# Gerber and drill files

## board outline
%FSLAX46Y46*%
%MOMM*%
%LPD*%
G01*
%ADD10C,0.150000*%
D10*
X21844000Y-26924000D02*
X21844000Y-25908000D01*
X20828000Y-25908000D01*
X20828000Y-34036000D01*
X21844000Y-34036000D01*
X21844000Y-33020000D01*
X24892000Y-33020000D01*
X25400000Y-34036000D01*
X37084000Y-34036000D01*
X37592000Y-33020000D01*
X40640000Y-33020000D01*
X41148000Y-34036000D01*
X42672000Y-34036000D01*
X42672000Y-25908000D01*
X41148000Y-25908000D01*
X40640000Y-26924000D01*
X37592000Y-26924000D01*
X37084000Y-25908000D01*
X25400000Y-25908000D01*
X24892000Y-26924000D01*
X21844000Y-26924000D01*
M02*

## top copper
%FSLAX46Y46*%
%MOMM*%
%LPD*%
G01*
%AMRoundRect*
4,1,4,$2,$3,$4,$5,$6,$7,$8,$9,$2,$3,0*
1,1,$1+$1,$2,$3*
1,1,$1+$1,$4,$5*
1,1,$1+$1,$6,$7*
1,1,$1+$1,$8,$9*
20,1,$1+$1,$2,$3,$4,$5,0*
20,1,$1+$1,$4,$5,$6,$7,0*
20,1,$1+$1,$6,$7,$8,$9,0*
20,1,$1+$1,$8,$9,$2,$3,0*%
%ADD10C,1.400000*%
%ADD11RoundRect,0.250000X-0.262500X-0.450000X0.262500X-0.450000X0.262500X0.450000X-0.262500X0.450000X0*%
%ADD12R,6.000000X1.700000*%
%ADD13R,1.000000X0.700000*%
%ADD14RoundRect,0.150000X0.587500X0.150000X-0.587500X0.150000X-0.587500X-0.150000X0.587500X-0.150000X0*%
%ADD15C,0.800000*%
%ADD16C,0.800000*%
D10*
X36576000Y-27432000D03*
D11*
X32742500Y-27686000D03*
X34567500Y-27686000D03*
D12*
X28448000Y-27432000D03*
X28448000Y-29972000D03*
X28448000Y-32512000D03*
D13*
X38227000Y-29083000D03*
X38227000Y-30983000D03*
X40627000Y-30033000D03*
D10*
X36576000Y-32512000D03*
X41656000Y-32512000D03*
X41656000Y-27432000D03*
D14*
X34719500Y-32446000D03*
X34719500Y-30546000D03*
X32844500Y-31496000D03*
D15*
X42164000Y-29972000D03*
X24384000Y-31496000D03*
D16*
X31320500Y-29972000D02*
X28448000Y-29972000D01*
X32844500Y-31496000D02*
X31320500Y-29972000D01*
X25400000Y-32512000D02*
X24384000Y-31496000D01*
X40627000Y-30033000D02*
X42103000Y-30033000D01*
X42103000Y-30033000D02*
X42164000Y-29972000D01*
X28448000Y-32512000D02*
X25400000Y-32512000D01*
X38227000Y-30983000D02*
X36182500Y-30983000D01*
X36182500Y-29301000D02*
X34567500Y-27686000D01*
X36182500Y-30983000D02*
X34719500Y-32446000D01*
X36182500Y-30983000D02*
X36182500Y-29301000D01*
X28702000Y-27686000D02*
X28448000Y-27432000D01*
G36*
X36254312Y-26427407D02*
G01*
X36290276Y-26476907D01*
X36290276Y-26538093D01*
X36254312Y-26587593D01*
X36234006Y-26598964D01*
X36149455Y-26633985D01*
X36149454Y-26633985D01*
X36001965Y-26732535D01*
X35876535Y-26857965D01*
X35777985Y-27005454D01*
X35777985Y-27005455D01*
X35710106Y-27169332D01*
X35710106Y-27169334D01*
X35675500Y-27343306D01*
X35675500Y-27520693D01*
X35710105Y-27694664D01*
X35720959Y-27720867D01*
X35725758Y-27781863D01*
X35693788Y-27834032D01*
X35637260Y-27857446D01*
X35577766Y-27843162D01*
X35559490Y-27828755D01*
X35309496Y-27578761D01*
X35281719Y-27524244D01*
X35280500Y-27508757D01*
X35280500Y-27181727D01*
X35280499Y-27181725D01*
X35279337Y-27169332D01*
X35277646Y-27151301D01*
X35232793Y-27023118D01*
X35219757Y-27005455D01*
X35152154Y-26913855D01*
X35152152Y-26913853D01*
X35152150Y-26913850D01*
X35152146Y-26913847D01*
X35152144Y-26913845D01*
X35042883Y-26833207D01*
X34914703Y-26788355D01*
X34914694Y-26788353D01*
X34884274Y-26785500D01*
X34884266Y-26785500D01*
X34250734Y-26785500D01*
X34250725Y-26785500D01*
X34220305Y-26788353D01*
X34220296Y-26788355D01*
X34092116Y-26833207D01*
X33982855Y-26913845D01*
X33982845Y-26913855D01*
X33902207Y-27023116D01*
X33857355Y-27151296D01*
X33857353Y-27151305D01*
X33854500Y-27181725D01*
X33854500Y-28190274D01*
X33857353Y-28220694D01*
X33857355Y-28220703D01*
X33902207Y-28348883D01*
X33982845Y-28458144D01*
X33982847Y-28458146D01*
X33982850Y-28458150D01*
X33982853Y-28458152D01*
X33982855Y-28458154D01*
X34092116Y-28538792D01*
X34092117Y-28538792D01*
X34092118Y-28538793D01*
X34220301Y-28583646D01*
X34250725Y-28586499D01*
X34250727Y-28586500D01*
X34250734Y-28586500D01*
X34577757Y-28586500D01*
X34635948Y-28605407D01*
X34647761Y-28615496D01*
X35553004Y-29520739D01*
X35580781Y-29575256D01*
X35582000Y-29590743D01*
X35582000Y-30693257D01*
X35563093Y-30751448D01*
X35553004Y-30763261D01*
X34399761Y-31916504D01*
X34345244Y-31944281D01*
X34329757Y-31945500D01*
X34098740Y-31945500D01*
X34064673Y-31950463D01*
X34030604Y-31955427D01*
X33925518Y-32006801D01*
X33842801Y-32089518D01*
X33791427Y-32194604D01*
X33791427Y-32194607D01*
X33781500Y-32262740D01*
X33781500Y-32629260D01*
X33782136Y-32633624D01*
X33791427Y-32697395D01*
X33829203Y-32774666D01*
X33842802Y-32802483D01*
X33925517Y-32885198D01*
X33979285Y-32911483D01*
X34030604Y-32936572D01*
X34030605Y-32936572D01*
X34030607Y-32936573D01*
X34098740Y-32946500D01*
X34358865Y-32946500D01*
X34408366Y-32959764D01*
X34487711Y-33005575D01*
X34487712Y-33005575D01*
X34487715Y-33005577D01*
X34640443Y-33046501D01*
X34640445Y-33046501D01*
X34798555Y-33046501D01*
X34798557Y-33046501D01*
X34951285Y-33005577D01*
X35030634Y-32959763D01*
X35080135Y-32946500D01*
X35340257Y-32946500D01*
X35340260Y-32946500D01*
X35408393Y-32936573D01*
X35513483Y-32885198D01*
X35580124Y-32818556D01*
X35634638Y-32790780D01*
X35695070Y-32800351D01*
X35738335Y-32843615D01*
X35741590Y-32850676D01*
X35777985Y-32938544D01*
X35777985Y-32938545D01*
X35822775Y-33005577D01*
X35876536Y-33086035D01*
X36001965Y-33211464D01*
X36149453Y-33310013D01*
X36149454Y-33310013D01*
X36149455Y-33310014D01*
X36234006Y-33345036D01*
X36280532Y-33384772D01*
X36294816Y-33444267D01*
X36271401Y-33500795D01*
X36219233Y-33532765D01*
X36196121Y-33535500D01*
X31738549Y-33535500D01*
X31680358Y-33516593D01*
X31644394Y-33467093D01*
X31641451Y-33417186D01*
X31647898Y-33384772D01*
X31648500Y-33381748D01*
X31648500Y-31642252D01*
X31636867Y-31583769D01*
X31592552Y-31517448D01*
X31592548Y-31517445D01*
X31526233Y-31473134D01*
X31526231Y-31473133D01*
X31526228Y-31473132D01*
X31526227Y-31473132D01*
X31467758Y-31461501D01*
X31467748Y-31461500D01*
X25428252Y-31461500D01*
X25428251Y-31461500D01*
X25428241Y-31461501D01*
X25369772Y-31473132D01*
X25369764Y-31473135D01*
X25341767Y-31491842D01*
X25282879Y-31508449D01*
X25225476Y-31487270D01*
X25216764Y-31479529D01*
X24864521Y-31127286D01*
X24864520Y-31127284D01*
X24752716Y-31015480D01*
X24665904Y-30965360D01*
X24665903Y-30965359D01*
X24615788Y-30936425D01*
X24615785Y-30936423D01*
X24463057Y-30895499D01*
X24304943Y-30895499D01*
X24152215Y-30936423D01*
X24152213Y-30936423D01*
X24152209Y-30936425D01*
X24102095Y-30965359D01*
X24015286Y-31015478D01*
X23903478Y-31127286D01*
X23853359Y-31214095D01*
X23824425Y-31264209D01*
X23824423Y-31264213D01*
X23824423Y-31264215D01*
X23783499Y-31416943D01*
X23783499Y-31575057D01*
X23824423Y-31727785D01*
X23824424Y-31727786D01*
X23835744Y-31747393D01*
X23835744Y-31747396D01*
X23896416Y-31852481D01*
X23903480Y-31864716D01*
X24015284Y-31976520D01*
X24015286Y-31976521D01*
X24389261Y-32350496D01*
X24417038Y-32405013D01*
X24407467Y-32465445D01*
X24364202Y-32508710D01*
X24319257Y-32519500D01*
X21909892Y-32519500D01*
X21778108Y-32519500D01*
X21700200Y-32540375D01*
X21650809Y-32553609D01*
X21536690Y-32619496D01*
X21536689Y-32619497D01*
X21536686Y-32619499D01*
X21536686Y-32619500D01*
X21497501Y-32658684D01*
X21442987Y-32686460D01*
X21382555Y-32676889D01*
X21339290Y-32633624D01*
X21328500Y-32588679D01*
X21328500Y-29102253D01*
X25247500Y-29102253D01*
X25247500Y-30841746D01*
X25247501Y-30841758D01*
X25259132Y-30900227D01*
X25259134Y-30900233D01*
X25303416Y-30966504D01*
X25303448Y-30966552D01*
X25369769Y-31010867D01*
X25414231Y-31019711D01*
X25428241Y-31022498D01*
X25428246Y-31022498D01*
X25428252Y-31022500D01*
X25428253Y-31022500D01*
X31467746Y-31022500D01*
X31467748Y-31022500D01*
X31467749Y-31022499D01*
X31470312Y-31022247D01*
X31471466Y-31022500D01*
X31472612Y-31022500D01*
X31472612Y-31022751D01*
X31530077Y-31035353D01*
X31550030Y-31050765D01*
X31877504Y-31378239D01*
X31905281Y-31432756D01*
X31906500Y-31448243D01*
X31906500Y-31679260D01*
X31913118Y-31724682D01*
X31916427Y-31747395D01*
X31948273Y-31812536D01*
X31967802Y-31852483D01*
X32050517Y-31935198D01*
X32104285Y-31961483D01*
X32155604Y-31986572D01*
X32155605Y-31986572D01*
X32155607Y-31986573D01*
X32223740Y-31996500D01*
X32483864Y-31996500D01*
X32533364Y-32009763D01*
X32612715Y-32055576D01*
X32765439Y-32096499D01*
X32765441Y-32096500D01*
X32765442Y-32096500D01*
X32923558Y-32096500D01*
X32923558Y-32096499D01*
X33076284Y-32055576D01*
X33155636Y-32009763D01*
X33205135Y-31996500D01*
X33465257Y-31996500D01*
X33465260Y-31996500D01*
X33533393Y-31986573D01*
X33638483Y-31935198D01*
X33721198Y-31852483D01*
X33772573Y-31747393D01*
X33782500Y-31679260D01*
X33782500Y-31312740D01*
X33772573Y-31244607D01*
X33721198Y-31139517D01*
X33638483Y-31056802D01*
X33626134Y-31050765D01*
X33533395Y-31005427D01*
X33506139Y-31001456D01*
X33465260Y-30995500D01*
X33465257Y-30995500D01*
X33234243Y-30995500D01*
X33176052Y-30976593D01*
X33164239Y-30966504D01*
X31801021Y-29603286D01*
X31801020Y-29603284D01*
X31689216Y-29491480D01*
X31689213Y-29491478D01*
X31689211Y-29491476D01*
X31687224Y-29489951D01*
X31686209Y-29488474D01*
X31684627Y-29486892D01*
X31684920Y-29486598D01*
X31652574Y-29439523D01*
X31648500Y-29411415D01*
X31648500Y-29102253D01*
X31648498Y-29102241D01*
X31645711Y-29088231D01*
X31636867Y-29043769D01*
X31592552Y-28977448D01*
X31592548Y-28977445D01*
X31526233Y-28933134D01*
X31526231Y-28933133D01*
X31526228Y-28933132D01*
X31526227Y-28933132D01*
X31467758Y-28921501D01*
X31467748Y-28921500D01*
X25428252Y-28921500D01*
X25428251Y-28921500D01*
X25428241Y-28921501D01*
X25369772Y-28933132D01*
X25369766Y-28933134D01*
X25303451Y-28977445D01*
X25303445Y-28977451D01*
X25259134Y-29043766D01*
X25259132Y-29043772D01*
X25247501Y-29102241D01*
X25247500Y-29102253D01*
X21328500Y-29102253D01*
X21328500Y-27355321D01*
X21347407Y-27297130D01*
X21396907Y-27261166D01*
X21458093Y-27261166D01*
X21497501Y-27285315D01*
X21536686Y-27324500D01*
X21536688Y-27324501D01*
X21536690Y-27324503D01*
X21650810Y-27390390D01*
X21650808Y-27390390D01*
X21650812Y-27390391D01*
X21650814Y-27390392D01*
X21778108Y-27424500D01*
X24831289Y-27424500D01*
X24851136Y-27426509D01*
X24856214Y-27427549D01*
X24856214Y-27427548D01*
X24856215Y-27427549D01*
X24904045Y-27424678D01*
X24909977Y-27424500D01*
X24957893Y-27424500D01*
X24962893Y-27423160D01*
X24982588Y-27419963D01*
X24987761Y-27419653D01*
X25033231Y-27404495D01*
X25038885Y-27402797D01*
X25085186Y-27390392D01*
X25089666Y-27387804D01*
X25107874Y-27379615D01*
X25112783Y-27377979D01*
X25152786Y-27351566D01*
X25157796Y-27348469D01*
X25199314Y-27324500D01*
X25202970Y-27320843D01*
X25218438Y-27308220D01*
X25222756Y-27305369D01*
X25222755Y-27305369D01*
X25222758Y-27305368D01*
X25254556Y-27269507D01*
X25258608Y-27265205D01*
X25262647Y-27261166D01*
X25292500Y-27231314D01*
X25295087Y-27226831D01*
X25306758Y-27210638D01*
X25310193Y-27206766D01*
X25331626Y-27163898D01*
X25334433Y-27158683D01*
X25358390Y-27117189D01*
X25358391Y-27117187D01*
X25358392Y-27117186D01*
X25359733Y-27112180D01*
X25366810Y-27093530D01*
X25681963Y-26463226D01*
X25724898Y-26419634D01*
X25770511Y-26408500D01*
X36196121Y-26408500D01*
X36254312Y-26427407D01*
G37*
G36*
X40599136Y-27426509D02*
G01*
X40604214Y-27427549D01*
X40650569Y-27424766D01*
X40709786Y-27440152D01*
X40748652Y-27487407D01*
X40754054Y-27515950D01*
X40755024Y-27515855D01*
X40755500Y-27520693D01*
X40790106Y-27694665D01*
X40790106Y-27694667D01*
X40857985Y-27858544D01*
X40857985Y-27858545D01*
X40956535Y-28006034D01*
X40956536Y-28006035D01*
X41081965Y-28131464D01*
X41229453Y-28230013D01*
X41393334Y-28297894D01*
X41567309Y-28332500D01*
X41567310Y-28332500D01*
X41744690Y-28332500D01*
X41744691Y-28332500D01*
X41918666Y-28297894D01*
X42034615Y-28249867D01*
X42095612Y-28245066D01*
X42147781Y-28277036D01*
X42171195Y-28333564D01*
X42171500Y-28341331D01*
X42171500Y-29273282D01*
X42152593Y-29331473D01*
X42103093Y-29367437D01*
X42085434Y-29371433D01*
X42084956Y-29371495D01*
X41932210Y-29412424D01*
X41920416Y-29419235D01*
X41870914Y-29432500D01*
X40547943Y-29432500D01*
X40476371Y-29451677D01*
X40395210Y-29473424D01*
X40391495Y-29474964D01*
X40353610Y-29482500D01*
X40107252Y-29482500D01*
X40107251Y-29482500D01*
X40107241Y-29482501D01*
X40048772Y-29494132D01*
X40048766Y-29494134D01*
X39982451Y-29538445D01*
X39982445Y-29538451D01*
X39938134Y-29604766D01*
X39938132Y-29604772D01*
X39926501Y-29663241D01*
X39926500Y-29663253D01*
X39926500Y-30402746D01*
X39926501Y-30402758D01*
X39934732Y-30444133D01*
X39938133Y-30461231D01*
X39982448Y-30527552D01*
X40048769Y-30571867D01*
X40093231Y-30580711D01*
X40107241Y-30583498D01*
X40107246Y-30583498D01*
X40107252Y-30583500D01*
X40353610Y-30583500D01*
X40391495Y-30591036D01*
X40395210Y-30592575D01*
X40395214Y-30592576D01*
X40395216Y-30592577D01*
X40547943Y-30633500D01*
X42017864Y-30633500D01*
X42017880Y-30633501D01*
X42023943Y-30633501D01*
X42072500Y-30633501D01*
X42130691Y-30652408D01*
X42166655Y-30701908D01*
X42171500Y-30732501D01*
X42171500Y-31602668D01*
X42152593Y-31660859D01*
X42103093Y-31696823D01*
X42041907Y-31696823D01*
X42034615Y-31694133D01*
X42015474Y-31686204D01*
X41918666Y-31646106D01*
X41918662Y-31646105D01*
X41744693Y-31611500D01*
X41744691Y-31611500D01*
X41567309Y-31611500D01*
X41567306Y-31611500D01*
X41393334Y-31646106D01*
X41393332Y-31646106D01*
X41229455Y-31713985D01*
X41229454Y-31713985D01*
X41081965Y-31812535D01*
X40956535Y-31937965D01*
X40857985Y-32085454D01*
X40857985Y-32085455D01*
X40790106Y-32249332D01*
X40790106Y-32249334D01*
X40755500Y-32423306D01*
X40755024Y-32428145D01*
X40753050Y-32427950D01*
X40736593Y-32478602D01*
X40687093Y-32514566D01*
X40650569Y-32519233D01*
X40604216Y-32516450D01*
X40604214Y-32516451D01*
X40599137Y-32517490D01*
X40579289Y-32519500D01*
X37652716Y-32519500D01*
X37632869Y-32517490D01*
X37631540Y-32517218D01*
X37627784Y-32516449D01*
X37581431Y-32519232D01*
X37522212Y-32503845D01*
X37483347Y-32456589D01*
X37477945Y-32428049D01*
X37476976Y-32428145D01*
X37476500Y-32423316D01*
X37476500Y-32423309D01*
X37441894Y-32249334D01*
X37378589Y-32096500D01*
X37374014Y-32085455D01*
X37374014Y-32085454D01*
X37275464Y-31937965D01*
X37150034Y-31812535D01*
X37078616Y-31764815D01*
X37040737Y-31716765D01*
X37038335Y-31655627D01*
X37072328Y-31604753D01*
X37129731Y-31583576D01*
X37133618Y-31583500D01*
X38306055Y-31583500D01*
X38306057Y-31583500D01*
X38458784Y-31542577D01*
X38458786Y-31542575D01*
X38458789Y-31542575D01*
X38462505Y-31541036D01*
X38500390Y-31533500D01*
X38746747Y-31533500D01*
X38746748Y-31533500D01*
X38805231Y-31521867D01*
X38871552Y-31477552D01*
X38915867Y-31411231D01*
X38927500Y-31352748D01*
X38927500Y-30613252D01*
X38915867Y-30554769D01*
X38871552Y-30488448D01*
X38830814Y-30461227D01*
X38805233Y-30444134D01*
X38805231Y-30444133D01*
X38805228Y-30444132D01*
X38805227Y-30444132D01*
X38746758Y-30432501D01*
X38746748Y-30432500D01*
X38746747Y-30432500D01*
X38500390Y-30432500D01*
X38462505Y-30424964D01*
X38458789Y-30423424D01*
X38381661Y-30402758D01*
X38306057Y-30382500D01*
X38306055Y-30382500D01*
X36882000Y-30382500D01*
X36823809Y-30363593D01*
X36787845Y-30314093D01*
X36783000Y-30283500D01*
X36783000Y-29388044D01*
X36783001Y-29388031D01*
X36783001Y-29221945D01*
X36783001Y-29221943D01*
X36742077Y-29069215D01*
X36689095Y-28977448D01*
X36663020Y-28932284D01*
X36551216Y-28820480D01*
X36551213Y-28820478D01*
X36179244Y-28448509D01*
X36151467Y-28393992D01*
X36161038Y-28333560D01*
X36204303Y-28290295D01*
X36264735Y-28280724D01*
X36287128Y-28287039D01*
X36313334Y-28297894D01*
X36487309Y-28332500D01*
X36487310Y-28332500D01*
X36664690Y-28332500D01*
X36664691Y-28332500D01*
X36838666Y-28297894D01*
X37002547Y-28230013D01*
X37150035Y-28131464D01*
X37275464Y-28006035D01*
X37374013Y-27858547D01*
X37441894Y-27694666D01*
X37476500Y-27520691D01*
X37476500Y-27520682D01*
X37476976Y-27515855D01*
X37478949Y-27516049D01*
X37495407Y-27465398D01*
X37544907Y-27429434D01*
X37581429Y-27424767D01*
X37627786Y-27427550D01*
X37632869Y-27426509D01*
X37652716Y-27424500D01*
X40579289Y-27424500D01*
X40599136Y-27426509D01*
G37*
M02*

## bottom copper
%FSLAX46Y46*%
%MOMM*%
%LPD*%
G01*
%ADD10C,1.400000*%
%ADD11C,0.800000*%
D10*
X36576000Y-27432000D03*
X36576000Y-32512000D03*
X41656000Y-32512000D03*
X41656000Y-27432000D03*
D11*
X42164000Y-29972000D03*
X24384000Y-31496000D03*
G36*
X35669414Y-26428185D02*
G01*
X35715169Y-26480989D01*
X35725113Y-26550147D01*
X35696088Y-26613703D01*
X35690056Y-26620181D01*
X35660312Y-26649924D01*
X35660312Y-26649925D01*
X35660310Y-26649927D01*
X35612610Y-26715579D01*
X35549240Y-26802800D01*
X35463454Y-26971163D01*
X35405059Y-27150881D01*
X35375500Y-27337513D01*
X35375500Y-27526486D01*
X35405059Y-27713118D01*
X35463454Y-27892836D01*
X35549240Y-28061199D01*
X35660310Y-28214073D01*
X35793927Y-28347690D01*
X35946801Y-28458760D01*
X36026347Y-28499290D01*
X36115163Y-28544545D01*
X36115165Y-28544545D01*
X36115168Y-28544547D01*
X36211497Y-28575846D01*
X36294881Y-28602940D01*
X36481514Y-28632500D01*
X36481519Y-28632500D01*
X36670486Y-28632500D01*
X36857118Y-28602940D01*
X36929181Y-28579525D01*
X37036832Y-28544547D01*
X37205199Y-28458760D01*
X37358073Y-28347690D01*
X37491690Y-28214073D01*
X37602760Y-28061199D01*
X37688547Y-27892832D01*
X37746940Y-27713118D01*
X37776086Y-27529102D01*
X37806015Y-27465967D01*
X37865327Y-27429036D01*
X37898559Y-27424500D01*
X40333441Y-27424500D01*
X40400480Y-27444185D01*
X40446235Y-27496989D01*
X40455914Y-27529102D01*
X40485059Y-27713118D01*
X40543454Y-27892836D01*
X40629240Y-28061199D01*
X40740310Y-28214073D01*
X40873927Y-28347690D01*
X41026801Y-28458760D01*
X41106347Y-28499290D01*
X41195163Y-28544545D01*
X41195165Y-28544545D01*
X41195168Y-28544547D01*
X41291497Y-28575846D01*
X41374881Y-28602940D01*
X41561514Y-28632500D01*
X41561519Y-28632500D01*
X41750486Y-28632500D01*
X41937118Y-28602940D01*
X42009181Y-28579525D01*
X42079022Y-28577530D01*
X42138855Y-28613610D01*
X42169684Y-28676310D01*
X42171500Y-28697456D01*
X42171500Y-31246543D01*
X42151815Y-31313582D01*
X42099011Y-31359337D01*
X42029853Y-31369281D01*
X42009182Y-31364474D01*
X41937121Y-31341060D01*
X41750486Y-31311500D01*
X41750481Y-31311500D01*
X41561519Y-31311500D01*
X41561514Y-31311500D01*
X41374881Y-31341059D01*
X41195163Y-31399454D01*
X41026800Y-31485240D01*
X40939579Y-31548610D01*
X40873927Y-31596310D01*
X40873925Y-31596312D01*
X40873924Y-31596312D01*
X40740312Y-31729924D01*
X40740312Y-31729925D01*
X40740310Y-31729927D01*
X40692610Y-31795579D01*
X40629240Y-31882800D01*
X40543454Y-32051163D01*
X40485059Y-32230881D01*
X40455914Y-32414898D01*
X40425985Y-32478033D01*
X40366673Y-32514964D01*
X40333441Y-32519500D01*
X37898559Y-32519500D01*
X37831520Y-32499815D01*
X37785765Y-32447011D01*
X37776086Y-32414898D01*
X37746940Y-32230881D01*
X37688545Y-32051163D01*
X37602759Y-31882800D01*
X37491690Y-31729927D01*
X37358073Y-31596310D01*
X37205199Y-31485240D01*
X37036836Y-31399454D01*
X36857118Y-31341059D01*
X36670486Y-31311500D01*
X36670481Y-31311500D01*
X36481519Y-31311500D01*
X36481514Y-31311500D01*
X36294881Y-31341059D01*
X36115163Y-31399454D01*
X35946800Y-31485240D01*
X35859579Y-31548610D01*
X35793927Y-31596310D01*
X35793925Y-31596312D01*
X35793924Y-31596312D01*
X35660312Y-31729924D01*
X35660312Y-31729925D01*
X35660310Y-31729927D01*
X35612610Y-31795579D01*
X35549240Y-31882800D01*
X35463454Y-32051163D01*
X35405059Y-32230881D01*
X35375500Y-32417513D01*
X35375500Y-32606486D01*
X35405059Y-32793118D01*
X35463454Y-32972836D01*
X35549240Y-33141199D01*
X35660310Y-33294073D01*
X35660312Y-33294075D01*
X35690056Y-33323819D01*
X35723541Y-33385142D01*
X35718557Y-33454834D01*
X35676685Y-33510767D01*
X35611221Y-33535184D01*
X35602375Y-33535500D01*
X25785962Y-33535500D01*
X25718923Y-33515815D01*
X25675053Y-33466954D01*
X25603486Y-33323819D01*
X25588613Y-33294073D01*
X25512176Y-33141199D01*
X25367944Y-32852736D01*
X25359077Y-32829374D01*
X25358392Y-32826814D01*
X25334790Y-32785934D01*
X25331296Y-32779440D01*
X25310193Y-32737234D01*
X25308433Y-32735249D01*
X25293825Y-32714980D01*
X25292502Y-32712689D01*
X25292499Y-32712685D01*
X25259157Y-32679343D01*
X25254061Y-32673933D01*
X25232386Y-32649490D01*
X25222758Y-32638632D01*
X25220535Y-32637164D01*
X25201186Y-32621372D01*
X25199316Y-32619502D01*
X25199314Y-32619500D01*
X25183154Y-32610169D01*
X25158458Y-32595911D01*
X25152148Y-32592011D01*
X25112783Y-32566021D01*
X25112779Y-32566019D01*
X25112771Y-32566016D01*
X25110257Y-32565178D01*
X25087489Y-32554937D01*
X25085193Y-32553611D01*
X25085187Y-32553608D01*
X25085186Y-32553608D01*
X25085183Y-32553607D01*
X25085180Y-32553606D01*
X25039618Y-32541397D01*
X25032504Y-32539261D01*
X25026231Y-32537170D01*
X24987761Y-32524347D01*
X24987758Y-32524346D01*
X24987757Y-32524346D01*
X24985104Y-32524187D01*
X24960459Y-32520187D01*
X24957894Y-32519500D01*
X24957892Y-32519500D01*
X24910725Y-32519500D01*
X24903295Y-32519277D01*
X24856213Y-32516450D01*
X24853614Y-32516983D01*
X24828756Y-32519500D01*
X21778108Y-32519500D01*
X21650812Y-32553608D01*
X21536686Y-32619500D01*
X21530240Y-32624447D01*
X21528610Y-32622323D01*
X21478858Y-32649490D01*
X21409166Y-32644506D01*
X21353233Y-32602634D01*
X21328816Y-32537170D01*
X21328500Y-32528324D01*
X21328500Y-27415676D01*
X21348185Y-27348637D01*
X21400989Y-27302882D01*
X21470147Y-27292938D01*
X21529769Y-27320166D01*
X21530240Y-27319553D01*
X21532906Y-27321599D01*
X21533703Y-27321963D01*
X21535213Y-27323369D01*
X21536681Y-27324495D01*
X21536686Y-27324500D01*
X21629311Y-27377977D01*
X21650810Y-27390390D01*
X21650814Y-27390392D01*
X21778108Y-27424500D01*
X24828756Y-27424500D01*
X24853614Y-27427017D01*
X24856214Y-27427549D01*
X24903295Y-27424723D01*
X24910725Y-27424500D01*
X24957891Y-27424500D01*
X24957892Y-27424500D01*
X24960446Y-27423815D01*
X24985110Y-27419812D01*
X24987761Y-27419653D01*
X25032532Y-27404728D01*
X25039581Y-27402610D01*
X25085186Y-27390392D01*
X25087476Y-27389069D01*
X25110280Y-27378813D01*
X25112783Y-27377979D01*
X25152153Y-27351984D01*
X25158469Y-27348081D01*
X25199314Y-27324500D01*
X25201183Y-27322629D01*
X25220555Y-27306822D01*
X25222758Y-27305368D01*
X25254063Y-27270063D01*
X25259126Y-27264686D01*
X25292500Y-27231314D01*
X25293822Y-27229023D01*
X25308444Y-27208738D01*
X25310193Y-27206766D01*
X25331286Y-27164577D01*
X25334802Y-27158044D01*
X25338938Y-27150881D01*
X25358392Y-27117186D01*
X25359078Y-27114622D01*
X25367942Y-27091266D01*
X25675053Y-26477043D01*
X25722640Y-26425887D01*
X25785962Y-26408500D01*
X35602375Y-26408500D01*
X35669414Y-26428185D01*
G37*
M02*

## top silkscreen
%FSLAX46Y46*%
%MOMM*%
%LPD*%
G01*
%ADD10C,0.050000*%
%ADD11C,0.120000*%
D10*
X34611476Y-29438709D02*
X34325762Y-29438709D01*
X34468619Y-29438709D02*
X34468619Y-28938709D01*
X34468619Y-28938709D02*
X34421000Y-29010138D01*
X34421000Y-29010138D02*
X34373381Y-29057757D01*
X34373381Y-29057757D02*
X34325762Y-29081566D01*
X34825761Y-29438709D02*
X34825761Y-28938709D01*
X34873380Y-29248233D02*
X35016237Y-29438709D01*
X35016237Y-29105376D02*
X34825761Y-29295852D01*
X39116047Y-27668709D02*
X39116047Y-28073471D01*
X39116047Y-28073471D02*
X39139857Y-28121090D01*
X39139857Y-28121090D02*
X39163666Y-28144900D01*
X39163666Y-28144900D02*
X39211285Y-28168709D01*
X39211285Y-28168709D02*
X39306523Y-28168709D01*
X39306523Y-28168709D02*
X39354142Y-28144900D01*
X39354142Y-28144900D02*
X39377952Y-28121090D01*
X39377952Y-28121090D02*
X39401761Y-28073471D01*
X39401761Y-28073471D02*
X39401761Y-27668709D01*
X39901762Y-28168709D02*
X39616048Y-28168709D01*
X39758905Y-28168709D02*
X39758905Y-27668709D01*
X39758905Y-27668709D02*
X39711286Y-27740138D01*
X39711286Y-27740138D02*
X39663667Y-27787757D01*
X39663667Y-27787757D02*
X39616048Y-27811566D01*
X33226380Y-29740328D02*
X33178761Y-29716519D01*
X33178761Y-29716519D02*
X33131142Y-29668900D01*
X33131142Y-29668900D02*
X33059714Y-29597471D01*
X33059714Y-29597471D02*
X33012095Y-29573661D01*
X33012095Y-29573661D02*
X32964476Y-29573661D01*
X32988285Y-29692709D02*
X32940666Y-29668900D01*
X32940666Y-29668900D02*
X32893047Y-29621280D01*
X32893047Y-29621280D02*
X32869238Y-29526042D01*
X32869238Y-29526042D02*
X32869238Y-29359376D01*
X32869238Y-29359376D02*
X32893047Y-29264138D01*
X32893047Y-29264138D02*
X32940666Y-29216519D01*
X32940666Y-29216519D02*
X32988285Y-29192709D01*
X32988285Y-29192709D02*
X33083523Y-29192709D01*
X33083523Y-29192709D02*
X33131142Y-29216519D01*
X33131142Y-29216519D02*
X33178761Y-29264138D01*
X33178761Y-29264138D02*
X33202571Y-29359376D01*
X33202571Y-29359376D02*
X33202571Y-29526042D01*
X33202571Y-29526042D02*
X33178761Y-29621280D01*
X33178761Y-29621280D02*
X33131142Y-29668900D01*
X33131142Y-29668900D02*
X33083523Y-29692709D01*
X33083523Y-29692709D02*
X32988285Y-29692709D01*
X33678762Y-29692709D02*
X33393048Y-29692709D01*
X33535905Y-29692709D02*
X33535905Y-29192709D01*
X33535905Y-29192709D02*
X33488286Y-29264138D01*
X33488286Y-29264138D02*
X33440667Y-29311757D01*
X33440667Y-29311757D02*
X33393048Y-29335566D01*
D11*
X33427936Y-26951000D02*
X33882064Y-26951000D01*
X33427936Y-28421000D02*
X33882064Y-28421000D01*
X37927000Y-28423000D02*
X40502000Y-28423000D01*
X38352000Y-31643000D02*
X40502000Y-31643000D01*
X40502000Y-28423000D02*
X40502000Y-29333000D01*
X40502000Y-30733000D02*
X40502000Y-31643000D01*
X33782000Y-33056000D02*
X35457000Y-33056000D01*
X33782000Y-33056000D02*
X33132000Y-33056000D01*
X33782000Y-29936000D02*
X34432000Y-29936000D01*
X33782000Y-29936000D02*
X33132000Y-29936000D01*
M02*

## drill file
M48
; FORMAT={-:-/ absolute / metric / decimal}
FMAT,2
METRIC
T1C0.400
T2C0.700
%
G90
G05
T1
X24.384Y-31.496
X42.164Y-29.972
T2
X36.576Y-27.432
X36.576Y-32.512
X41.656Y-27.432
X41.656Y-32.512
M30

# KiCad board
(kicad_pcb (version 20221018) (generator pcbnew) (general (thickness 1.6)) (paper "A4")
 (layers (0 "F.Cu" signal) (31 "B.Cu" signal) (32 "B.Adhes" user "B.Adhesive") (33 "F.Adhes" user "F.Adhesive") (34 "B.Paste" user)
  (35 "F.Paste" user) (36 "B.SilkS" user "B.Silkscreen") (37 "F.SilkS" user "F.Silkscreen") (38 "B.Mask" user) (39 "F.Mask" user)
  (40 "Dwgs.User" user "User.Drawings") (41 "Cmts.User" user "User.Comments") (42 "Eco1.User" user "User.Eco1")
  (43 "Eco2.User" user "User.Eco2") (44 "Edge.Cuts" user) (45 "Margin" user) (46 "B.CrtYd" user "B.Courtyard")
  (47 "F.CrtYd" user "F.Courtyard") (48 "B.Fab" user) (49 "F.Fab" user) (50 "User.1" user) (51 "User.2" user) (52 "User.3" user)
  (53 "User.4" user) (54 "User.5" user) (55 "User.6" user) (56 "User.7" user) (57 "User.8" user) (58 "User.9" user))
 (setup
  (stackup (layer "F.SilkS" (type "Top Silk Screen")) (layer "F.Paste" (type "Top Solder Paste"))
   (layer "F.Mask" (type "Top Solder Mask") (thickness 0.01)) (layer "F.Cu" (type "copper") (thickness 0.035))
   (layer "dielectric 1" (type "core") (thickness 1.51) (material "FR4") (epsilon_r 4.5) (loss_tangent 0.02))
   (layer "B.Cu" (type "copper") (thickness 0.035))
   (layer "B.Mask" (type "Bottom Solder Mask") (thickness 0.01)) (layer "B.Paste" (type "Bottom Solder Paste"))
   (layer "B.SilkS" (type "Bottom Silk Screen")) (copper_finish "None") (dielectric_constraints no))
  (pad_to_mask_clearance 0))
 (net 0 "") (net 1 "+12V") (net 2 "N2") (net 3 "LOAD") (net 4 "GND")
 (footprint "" (layer "F.Cu") (at 36.576 27.432)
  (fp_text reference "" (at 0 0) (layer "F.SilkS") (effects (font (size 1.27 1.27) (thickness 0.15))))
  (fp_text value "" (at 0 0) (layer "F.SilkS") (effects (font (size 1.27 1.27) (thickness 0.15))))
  (pad "1" thru_hole circle (at 0 0) (size 1.4 1.4) (drill 0.7) (layers "*.Cu" "*.Mask")))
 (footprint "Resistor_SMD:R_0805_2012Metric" (layer "F.Cu") (at 33.655 27.686)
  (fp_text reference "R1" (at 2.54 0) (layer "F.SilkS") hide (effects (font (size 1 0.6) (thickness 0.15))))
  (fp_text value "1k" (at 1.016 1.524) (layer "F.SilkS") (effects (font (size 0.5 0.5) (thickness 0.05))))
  (fp_line (start -0.227064 -0.735) (end 0.227064 -0.735) (stroke (width 0.12) (type solid)) (layer "F.SilkS"))
  (fp_line (start -0.227064 0.735) (end 0.227064 0.735) (stroke (width 0.12) (type solid)) (layer "F.SilkS"))
  (pad "1" smd roundrect (at -0.9125 0) (size 1.025 1.4) (layers "F.Cu" "F.Paste" "F.Mask") (roundrect_rratio 0.243902) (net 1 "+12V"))
  (pad "2" smd roundrect (at 0.9125 0) (size 1.025 1.4) (layers "F.Cu" "F.Paste" "F.Mask") (roundrect_rratio 0.243902) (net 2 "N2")))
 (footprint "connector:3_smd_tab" (layer "F.Cu") (at 28.448 27.432)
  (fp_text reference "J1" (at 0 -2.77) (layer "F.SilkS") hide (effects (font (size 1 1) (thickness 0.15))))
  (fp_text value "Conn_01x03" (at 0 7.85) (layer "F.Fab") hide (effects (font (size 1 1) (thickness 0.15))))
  (pad "1" smd rect (at 0 0) (size 6 1.7) (layers "F.Cu" "F.Paste" "F.Mask") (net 1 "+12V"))
  (pad "2" smd rect (at 0 2.54) (size 6 1.7) (layers "F.Cu" "F.Paste" "F.Mask") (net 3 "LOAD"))
  (pad "3" smd rect (at 0 5.08) (size 6 1.7) (layers "F.Cu" "F.Paste" "F.Mask") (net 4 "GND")))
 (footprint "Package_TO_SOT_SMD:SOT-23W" (layer "F.Cu") (at 39.427 30.033)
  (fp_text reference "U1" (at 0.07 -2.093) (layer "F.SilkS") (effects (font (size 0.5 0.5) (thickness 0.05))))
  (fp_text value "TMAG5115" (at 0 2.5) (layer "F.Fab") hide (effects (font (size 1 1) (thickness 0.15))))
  (fp_line (start -1.5 -1.61) (end 1.075 -1.61) (stroke (width 0.12) (type solid)) (layer "F.SilkS"))
  (fp_line (start -1.075 1.61) (end 1.075 1.61) (stroke (width 0.12) (type solid)) (layer "F.SilkS"))
  (fp_line (start 1.075 -1.61) (end 1.075 -0.7) (stroke (width 0.12) (type solid)) (layer "F.SilkS"))
  (fp_line (start 1.075 0.7) (end 1.075 1.61) (stroke (width 0.12) (type solid)) (layer "F.SilkS"))
  (pad "1" smd rect (at -1.2 -0.95) (size 1 0.7) (layers "F.Cu" "F.Paste" "F.Mask") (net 1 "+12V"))
  (pad "2" smd rect (at -1.2 0.95) (size 1 0.7) (layers "F.Cu" "F.Paste" "F.Mask") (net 2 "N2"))
  (pad "3" smd rect (at 1.2 0) (size 1 0.7) (layers "F.Cu" "F.Paste" "F.Mask") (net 4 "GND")))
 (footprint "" (layer "F.Cu") (at 36.576 32.512)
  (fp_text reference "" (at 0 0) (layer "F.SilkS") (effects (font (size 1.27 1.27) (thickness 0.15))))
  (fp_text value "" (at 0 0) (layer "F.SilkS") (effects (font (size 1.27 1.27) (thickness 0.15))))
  (pad "1" thru_hole circle (at 0 0) (size 1.4 1.4) (drill 0.7) (layers "*.Cu" "*.Mask")))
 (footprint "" (layer "F.Cu") (at 41.656 32.512)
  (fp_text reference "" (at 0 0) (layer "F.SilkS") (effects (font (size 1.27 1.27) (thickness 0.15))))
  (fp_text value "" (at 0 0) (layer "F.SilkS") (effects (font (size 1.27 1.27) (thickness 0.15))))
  (pad "1" thru_hole circle (at 0 0) (size 1.4 1.4) (drill 0.7) (layers "*.Cu" "*.Mask")))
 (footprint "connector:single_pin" (layer "F.Cu") (at 41.656 27.432)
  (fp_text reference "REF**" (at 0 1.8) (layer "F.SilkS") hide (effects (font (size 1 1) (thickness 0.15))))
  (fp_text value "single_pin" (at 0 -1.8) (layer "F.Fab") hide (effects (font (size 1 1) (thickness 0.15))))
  (pad "1" thru_hole circle (at 0 0) (size 1.4 1.4) (drill 0.7) (layers "*.Cu" "*.Mask")))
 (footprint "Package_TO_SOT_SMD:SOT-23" (layer "F.Cu") (at 33.782 31.496 180)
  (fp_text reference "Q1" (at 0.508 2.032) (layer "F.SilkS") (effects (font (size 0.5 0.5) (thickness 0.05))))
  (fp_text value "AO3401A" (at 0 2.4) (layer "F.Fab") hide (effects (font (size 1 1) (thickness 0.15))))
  (fp_line (start 0 -1.56) (end -1.675 -1.56) (stroke (width 0.12) (type solid)) (layer "F.SilkS"))
  (fp_line (start 0 -1.56) (end 0.65 -1.56) (stroke (width 0.12) (type solid)) (layer "F.SilkS"))
  (fp_line (start 0 1.56) (end -0.65 1.56) (stroke (width 0.12) (type solid)) (layer "F.SilkS"))
  (fp_line (start 0 1.56) (end 0.65 1.56) (stroke (width 0.12) (type solid)) (layer "F.SilkS"))
  (pad "1" smd roundrect (at -0.9375 -0.95 180) (size 1.475 0.6) (layers "F.Cu" "F.Paste" "F.Mask") (roundrect_rratio 0.25) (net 2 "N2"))
  (pad "2" smd roundrect (at -0.9375 0.95 180) (size 1.475 0.6) (layers "F.Cu" "F.Paste" "F.Mask") (roundrect_rratio 0.25) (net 1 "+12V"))
  (pad "3" smd roundrect (at 0.9375 0 180) (size 1.475 0.6) (layers "F.Cu" "F.Paste" "F.Mask") (roundrect_rratio 0.25) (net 3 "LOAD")))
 (gr_poly
  (pts (xy 21.844 26.924) (xy 21.844 25.908) (xy 20.828 25.908) (xy 20.828 34.036) (xy 21.844 34.036) (xy 21.844 33.02) (xy 24.892 33.02)
   (xy 25.4 34.036) (xy 37.084 34.036) (xy 37.592 33.02) (xy 40.64 33.02) (xy 41.148 34.036) (xy 42.672 34.036) (xy 42.672 25.908)
   (xy 41.148 25.908) (xy 40.64 26.924) (xy 37.592 26.924) (xy 37.084 25.908) (xy 25.4 25.908) (xy 24.892 26.924))
  (stroke (width 0.15) (type solid)) (fill none) (layer "Edge.Cuts"))
 (segment (start 31.3205 29.972) (end 28.448 29.972) (width 0.8) (layer "F.Cu") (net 3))
 (segment (start 32.8445 31.496) (end 31.3205 29.972) (width 0.8) (layer "F.Cu") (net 3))
 (segment (start 25.4 32.512) (end 24.384 31.496) (width 0.8) (layer "F.Cu") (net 4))
 (segment (start 40.627 30.033) (end 42.103 30.033) (width 0.8) (layer "F.Cu") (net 4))
 (segment (start 42.103 30.033) (end 42.164 29.972) (width 0.8) (layer "F.Cu") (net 4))
 (segment (start 28.448 32.512) (end 25.4 32.512) (width 0.8) (layer "F.Cu") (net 4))
 (via (at 42.164 29.972) (size 0.8) (drill 0.4) (layers "F.Cu" "B.Cu") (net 4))
 (via (at 24.384 31.496) (size 0.8) (drill 0.4) (layers "F.Cu" "B.Cu") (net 4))
 (segment (start 38.227 30.983) (end 36.1825 30.983) (width 0.8) (layer "F.Cu") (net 2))
 (segment (start 36.1825 29.301) (end 34.5675 27.686) (width 0.8) (layer "F.Cu") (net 2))
 (segment (start 36.1825 30.983) (end 34.7195 32.446) (width 0.8) (layer "F.Cu") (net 2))
 (segment (start 36.1825 30.983) (end 36.1825 29.301) (width 0.8) (layer "F.Cu") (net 2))
 (segment (start 28.702 27.686) (end 28.448 27.432) (width 0.8) (layer "F.Cu") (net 1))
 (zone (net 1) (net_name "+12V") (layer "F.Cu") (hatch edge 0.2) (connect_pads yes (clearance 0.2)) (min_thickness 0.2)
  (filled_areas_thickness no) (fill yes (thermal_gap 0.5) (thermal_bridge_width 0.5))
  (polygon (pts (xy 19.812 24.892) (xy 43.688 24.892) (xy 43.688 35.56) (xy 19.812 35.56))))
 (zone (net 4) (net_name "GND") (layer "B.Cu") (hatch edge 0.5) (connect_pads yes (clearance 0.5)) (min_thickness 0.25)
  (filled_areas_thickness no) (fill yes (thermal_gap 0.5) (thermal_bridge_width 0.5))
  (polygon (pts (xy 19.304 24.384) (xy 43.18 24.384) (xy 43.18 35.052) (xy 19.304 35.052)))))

